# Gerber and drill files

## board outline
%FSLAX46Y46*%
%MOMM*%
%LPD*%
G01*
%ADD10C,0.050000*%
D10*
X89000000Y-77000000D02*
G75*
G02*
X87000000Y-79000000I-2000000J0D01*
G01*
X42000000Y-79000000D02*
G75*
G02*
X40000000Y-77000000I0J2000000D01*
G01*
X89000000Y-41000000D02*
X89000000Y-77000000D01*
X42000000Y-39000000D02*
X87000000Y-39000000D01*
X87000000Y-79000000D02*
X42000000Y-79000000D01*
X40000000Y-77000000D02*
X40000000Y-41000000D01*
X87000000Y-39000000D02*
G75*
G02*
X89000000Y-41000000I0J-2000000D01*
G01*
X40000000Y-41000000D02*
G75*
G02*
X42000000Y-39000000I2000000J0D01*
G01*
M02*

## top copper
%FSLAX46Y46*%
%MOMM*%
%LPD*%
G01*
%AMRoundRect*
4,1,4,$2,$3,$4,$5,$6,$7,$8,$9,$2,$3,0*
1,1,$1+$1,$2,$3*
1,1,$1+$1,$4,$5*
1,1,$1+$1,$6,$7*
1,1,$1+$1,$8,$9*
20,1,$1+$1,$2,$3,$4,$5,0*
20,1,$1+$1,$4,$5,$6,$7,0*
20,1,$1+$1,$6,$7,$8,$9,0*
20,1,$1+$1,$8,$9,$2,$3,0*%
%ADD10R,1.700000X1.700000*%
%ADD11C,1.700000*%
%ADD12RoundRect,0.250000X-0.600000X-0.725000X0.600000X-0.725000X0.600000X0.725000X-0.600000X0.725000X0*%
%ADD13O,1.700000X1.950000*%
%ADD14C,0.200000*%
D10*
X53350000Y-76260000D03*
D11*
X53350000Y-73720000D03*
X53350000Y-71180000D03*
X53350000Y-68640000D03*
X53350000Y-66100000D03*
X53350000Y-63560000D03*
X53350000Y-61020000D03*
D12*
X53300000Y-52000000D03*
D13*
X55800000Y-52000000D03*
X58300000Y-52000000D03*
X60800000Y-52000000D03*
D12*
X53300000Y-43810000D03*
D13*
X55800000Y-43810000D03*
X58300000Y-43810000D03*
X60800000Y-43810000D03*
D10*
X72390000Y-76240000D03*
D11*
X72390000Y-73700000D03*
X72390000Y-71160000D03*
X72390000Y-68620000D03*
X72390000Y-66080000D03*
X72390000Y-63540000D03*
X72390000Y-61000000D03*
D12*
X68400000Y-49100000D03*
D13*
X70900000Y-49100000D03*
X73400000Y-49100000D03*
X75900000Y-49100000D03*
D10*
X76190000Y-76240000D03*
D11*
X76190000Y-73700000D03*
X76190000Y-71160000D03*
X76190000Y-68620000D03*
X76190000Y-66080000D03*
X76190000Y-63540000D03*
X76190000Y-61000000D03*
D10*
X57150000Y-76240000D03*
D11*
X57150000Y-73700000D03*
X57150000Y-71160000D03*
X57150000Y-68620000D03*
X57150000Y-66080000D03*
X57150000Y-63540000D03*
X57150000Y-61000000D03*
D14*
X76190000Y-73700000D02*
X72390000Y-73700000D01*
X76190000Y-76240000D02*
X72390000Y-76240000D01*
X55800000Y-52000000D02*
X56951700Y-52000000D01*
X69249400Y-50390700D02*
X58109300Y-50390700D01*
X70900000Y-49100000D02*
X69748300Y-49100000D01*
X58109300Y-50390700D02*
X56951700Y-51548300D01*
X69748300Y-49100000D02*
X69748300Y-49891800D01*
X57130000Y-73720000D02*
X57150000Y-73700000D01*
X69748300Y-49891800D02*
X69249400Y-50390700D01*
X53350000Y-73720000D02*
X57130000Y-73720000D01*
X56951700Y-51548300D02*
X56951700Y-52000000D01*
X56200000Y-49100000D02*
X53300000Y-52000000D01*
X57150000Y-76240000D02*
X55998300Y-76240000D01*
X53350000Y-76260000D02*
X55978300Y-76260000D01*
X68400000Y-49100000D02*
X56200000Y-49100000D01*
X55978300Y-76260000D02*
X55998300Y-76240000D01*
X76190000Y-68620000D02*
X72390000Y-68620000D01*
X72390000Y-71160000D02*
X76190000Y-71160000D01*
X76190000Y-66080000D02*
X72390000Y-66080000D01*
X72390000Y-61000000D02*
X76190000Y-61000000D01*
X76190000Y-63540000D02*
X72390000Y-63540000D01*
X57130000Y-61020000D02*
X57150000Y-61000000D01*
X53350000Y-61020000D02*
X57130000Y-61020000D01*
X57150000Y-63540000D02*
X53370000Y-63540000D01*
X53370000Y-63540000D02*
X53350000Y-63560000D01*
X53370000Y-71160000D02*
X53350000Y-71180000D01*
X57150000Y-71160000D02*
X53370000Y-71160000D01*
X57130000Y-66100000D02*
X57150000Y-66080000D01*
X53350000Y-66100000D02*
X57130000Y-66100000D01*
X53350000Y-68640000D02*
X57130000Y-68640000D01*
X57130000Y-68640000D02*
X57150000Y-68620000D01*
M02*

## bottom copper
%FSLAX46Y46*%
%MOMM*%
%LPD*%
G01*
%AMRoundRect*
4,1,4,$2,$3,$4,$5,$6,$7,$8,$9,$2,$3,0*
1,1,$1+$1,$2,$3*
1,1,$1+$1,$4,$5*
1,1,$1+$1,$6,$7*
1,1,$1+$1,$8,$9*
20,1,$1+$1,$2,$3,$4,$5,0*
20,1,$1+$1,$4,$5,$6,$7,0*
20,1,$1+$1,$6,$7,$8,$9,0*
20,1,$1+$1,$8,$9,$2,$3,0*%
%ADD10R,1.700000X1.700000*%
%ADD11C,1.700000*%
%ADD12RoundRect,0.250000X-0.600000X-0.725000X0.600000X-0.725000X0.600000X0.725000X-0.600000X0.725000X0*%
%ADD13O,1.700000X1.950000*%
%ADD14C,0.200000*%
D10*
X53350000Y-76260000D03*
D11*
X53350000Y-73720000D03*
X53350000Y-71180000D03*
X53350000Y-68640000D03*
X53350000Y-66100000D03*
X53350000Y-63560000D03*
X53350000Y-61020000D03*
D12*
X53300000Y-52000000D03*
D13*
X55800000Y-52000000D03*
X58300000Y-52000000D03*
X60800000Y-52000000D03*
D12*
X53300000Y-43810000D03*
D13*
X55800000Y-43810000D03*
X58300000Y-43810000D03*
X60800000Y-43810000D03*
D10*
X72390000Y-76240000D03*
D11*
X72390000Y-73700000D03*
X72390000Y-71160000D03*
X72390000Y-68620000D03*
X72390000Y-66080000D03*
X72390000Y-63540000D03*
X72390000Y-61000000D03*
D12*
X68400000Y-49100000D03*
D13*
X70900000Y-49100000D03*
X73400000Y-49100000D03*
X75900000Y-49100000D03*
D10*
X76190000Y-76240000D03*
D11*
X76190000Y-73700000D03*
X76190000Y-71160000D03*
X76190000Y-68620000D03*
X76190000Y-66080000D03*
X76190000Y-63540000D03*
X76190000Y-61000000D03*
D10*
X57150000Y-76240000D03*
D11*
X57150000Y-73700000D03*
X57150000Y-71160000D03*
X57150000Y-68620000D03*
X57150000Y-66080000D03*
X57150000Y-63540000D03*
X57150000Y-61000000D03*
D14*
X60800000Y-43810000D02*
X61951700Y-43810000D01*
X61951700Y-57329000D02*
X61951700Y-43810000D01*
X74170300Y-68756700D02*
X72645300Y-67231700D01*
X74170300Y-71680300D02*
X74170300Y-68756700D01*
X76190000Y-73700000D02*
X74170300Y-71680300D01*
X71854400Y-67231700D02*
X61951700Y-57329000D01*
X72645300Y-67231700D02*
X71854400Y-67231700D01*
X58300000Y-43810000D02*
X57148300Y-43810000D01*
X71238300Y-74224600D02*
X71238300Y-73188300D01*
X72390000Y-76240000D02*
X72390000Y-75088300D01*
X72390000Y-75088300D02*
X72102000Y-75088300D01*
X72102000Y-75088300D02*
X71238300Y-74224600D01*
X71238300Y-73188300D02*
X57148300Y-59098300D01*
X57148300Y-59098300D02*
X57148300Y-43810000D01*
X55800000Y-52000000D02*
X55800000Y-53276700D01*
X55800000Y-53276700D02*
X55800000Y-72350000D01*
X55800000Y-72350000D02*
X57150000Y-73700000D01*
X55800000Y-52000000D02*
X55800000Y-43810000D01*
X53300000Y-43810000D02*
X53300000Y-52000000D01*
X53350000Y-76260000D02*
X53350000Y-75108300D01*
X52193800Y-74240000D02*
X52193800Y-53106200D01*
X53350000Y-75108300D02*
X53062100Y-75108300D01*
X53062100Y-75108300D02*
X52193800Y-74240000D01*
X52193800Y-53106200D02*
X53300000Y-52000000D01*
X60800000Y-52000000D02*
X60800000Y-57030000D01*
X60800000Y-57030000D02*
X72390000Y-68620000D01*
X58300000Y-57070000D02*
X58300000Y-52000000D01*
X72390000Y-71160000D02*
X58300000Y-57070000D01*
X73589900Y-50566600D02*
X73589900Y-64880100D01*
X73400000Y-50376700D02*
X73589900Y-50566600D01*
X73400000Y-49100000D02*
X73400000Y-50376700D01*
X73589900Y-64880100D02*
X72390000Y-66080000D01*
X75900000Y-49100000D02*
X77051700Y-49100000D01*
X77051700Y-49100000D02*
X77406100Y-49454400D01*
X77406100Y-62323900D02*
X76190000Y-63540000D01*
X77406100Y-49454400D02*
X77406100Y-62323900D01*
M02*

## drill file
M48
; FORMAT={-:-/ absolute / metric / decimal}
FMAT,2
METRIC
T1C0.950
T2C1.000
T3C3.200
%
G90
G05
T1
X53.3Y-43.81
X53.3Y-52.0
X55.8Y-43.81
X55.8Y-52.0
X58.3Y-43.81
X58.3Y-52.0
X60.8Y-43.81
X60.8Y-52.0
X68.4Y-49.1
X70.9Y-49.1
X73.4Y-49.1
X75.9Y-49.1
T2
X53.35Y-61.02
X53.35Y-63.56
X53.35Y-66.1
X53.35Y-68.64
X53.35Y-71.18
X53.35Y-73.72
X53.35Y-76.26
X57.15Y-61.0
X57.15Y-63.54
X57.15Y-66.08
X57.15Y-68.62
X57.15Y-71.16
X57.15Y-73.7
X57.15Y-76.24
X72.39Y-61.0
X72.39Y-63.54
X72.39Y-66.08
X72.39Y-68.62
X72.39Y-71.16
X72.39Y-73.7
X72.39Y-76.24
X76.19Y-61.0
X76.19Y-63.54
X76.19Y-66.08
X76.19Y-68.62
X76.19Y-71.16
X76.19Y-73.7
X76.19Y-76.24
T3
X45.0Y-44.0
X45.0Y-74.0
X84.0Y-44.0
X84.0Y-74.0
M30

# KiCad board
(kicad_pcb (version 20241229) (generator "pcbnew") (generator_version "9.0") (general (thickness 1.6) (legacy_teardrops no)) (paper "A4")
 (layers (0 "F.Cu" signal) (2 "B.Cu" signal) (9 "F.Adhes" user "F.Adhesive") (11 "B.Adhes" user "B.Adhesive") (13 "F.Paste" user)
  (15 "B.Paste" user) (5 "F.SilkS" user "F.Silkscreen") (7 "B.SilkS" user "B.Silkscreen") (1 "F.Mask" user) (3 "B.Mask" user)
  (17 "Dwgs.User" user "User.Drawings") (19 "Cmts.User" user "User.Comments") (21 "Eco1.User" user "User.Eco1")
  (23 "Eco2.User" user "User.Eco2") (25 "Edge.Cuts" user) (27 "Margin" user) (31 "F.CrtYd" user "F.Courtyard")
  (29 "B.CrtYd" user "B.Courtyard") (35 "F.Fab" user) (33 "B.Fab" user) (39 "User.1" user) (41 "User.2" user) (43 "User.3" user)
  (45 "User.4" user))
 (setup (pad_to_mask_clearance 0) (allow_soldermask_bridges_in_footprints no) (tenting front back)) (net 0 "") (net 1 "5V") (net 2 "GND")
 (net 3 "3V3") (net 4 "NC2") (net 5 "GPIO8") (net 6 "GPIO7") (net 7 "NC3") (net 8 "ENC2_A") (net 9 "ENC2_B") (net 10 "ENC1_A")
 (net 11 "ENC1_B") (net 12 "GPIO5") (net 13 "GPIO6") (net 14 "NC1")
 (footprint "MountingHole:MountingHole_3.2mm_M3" (layer "F.Cu") (at 84 44)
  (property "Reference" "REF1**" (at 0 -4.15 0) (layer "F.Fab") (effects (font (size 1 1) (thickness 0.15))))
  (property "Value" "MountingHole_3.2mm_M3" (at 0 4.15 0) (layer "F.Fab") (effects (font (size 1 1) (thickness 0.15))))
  (pad "" np_thru_hole circle (at 0 0) (size 3.2 3.2) (drill 3.2) (layers "*.Cu" "*.Mask")))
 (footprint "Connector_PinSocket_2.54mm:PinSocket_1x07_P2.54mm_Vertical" (layer "F.Cu") (at 53.35 76.26 180)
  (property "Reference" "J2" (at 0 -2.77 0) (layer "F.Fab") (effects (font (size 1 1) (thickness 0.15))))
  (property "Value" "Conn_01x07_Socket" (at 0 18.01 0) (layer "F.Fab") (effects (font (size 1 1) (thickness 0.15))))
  (pad "1" thru_hole rect (at 0 0 180) (size 1.7 1.7) (drill 1) (layers "*.Cu" "*.Mask") (remove_unused_layers no) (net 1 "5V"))
  (pad "2" thru_hole circle (at 0 2.54 180) (size 1.7 1.7) (drill 1) (layers "*.Cu" "*.Mask") (remove_unused_layers no) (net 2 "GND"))
  (pad "3" thru_hole circle (at 0 5.08 180) (size 1.7 1.7) (drill 1) (layers "*.Cu" "*.Mask") (remove_unused_layers no) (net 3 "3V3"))
  (pad "4" thru_hole circle (at 0 7.62 180) (size 1.7 1.7) (drill 1) (layers "*.Cu" "*.Mask") (remove_unused_layers no) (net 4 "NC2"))
  (pad "5" thru_hole circle (at 0 10.16 180) (size 1.7 1.7) (drill 1) (layers "*.Cu" "*.Mask") (remove_unused_layers no) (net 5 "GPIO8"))
  (pad "6" thru_hole circle (at 0 12.7 180) (size 1.7 1.7) (drill 1) (layers "*.Cu" "*.Mask") (remove_unused_layers no) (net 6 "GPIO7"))
  (pad "7" thru_hole circle (at 0 15.24 180) (size 1.7 1.7) (drill 1) (layers "*.Cu" "*.Mask") (remove_unused_layers no) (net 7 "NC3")))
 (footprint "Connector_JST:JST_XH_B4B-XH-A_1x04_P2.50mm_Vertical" (layer "F.Cu") (at 53.3 52)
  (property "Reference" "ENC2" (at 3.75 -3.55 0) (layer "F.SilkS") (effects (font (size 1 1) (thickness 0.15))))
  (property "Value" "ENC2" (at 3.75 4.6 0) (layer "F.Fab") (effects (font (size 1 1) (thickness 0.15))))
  (pad "1" thru_hole roundrect (at 0 0) (size 1.7 1.95) (drill 0.95) (layers "*.Cu" "*.Mask") (remove_unused_layers no)
   (roundrect_rratio 0.147059) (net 1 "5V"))
  (pad "2" thru_hole oval (at 2.5 0) (size 1.7 1.95) (drill 0.95) (layers "*.Cu" "*.Mask") (remove_unused_layers no) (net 2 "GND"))
  (pad "3" thru_hole oval (at 5 0) (size 1.7 1.95) (drill 0.95) (layers "*.Cu" "*.Mask") (remove_unused_layers no) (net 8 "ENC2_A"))
  (pad "4" thru_hole oval (at 7.5 0) (size 1.7 1.95) (drill 0.95) (layers "*.Cu" "*.Mask") (remove_unused_layers no) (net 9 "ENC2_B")))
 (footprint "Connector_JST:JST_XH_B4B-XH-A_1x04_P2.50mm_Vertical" (layer "F.Cu") (at 53.3 43.81)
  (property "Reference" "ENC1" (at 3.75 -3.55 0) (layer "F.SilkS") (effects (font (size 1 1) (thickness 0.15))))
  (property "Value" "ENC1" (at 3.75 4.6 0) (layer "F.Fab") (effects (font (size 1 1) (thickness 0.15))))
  (pad "1" thru_hole roundrect (at 0 0) (size 1.7 1.95) (drill 0.95) (layers "*.Cu" "*.Mask") (remove_unused_layers no)
   (roundrect_rratio 0.147059) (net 1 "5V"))
  (pad "2" thru_hole oval (at 2.5 0) (size 1.7 1.95) (drill 0.95) (layers "*.Cu" "*.Mask") (remove_unused_layers no) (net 2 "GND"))
  (pad "3" thru_hole oval (at 5 0) (size 1.7 1.95) (drill 0.95) (layers "*.Cu" "*.Mask") (remove_unused_layers no) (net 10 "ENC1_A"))
  (pad "4" thru_hole oval (at 7.5 0) (size 1.7 1.95) (drill 0.95) (layers "*.Cu" "*.Mask") (remove_unused_layers no) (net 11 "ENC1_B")))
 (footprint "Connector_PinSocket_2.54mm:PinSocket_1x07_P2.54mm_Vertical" (layer "F.Cu") (at 72.39 76.24 180)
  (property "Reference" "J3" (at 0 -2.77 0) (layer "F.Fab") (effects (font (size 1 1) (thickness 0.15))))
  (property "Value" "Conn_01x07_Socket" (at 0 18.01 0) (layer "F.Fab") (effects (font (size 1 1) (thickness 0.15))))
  (pad "1" thru_hole rect (at 0 0 180) (size 1.7 1.7) (drill 1) (layers "*.Cu" "*.Mask") (remove_unused_layers no) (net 10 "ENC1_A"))
  (pad "2" thru_hole circle (at 0 2.54 180) (size 1.7 1.7) (drill 1) (layers "*.Cu" "*.Mask") (remove_unused_layers no) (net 11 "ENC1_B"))
  (pad "3" thru_hole circle (at 0 5.08 180) (size 1.7 1.7) (drill 1) (layers "*.Cu" "*.Mask") (remove_unused_layers no) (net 8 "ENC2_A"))
  (pad "4" thru_hole circle (at 0 7.62 180) (size 1.7 1.7) (drill 1) (layers "*.Cu" "*.Mask") (remove_unused_layers no) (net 9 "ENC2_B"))
  (pad "5" thru_hole circle (at 0 10.16 180) (size 1.7 1.7) (drill 1) (layers "*.Cu" "*.Mask") (remove_unused_layers no) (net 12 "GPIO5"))
  (pad "6" thru_hole circle (at 0 12.7 180) (size 1.7 1.7) (drill 1) (layers "*.Cu" "*.Mask") (remove_unused_layers no) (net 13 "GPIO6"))
  (pad "7" thru_hole circle (at 0 15.24 180) (size 1.7 1.7) (drill 1) (layers "*.Cu" "*.Mask") (remove_unused_layers no) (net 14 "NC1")))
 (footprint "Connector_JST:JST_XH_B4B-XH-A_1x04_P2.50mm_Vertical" (layer "F.Cu") (at 68.4 49.1)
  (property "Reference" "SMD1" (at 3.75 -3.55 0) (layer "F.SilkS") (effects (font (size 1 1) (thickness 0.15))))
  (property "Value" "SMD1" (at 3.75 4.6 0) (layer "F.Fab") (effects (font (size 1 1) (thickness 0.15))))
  (pad "1" thru_hole roundrect (at 0 0) (size 1.7 1.95) (drill 0.95) (layers "*.Cu" "*.Mask") (remove_unused_layers no)
   (roundrect_rratio 0.147059) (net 1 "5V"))
  (pad "2" thru_hole oval (at 2.5 0) (size 1.7 1.95) (drill 0.95) (layers "*.Cu" "*.Mask") (remove_unused_layers no) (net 2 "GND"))
  (pad "3" thru_hole oval (at 5 0) (size 1.7 1.95) (drill 0.95) (layers "*.Cu" "*.Mask") (remove_unused_layers no) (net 12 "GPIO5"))
  (pad "4" thru_hole oval (at 7.5 0) (size 1.7 1.95) (drill 0.95) (layers "*.Cu" "*.Mask") (remove_unused_layers no) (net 13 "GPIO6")))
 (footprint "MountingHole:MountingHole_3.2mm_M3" (layer "F.Cu") (at 45 74)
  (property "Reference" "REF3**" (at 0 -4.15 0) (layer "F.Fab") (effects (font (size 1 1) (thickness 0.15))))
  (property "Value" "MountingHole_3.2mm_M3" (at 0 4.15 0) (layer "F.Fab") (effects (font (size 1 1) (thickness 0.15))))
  (pad "" np_thru_hole circle (at 0 0) (size 3.2 3.2) (drill 3.2) (layers "*.Cu" "*.Mask")))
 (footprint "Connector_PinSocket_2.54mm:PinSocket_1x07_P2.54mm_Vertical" (layer "F.Cu") (at 76.19 76.24 180)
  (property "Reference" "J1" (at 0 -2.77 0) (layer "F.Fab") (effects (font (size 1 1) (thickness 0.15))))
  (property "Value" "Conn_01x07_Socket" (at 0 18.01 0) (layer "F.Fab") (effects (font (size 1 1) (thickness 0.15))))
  (pad "1" thru_hole rect (at 0 0 180) (size 1.7 1.7) (drill 1) (layers "*.Cu" "*.Mask") (remove_unused_layers no) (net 10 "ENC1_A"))
  (pad "2" thru_hole circle (at 0 2.54 180) (size 1.7 1.7) (drill 1) (layers "*.Cu" "*.Mask") (remove_unused_layers no) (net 11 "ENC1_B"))
  (pad "3" thru_hole circle (at 0 5.08 180) (size 1.7 1.7) (drill 1) (layers "*.Cu" "*.Mask") (remove_unused_layers no) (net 8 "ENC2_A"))
  (pad "4" thru_hole circle (at 0 7.62 180) (size 1.7 1.7) (drill 1) (layers "*.Cu" "*.Mask") (remove_unused_layers no) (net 9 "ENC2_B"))
  (pad "5" thru_hole circle (at 0 10.16 180) (size 1.7 1.7) (drill 1) (layers "*.Cu" "*.Mask") (remove_unused_layers no) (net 12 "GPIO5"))
  (pad "6" thru_hole circle (at 0 12.7 180) (size 1.7 1.7) (drill 1) (layers "*.Cu" "*.Mask") (remove_unused_layers no) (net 13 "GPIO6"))
  (pad "7" thru_hole circle (at 0 15.24 180) (size 1.7 1.7) (drill 1) (layers "*.Cu" "*.Mask") (remove_unused_layers no) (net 14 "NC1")))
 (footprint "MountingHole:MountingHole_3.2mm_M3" (layer "F.Cu") (at 45 44)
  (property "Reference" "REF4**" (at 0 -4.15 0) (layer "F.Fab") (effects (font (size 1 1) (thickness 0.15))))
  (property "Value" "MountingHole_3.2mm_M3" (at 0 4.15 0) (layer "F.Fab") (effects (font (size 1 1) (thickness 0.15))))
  (pad "" np_thru_hole circle (at 0 0) (size 3.2 3.2) (drill 3.2) (layers "*.Cu" "*.Mask")))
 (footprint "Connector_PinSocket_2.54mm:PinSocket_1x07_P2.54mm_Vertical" (layer "F.Cu") (at 57.15 76.24 180)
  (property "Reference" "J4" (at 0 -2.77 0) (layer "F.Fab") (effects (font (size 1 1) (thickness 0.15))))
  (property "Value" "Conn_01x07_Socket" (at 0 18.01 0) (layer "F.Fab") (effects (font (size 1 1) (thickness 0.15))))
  (pad "1" thru_hole rect (at 0 0 180) (size 1.7 1.7) (drill 1) (layers "*.Cu" "*.Mask") (remove_unused_layers no) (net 1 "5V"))
  (pad "2" thru_hole circle (at 0 2.54 180) (size 1.7 1.7) (drill 1) (layers "*.Cu" "*.Mask") (remove_unused_layers no) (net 2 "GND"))
  (pad "3" thru_hole circle (at 0 5.08 180) (size 1.7 1.7) (drill 1) (layers "*.Cu" "*.Mask") (remove_unused_layers no) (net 3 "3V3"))
  (pad "4" thru_hole circle (at 0 7.62 180) (size 1.7 1.7) (drill 1) (layers "*.Cu" "*.Mask") (remove_unused_layers no) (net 4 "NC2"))
  (pad "5" thru_hole circle (at 0 10.16 180) (size 1.7 1.7) (drill 1) (layers "*.Cu" "*.Mask") (remove_unused_layers no) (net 5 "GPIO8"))
  (pad "6" thru_hole circle (at 0 12.7 180) (size 1.7 1.7) (drill 1) (layers "*.Cu" "*.Mask") (remove_unused_layers no) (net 6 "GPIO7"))
  (pad "7" thru_hole circle (at 0 15.24 180) (size 1.7 1.7) (drill 1) (layers "*.Cu" "*.Mask") (remove_unused_layers no) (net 7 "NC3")))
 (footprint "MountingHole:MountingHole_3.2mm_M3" (layer "F.Cu") (at 84 74)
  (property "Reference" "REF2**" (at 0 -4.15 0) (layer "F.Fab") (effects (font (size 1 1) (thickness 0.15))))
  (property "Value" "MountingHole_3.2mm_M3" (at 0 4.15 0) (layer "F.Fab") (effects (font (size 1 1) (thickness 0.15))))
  (pad "" np_thru_hole circle (at 0 0) (size 3.2 3.2) (drill 3.2) (layers "*.Cu" "*.Mask")))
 (gr_arc (start 89 77) (mid 88.414214 78.414214) (end 87 79) (stroke (width 0.05) (type default)) (layer "Edge.Cuts"))
 (gr_arc (start 42 79) (mid 40.585786 78.414214) (end 40 77) (stroke (width 0.05) (type default)) (layer "Edge.Cuts"))
 (gr_line (start 89 41) (end 89 77) (stroke (width 0.05) (type default)) (layer "Edge.Cuts"))
 (gr_line (start 42 39) (end 87 39) (stroke (width 0.05) (type default)) (layer "Edge.Cuts"))
 (gr_line (start 87 79) (end 42 79) (stroke (width 0.05) (type default)) (layer "Edge.Cuts"))
 (gr_line (start 40 77) (end 40 41) (stroke (width 0.05) (type default)) (layer "Edge.Cuts"))
 (gr_arc (start 87 39) (mid 88.414214 39.585786) (end 89 41) (stroke (width 0.05) (type default)) (layer "Edge.Cuts"))
 (gr_arc (start 40 41) (mid 40.585786 39.585786) (end 42 39) (stroke (width 0.05) (type default)) (layer "Edge.Cuts"))
 (segment (start 76.19 73.7) (end 72.39 73.7) (width 0.2) (layer "F.Cu") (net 11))
 (segment (start 60.8 43.81) (end 61.9517 43.81) (width 0.2) (layer "B.Cu") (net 11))
 (segment (start 61.9517 57.329) (end 61.9517 43.81) (width 0.2) (layer "B.Cu") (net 11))
 (segment (start 74.1703 68.7567) (end 72.6453 67.2317) (width 0.2) (layer "B.Cu") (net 11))
 (segment (start 74.1703 71.6803) (end 74.1703 68.7567) (width 0.2) (layer "B.Cu") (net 11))
 (segment (start 76.19 73.7) (end 74.1703 71.6803) (width 0.2) (layer "B.Cu") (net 11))
 (segment (start 71.8544 67.2317) (end 61.9517 57.329) (width 0.2) (layer "B.Cu") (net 11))
 (segment (start 72.6453 67.2317) (end 71.8544 67.2317) (width 0.2) (layer "B.Cu") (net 11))
 (segment (start 76.19 76.24) (end 72.39 76.24) (width 0.2) (layer "F.Cu") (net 10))
 (segment (start 58.3 43.81) (end 57.1483 43.81) (width 0.2) (layer "B.Cu") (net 10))
 (segment (start 71.2383 74.2246) (end 71.2383 73.1883) (width 0.2) (layer "B.Cu") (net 10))
 (segment (start 72.39 76.24) (end 72.39 75.0883) (width 0.2) (layer "B.Cu") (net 10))
 (segment (start 72.39 75.0883) (end 72.102 75.0883) (width 0.2) (layer "B.Cu") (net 10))
 (segment (start 72.102 75.0883) (end 71.2383 74.2246) (width 0.2) (layer "B.Cu") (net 10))
 (segment (start 71.2383 73.1883) (end 57.1483 59.0983) (width 0.2) (layer "B.Cu") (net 10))
 (segment (start 57.1483 59.0983) (end 57.1483 43.81) (width 0.2) (layer "B.Cu") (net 10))
 (segment (start 55.8 52) (end 56.9517 52) (width 0.2) (layer "F.Cu") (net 2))
 (segment (start 69.2494 50.3907) (end 58.1093 50.3907) (width 0.2) (layer "F.Cu") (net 2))
 (segment (start 70.9 49.1) (end 69.7483 49.1) (width 0.2) (layer "F.Cu") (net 2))
 (segment (start 58.1093 50.3907) (end 56.9517 51.5483) (width 0.2) (layer "F.Cu") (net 2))
 (segment (start 69.7483 49.1) (end 69.7483 49.8918) (width 0.2) (layer "F.Cu") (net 2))
 (segment (start 57.13 73.72) (end 57.15 73.7) (width 0.2) (layer "F.Cu") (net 2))
 (segment (start 69.7483 49.8918) (end 69.2494 50.3907) (width 0.2) (layer "F.Cu") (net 2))
 (segment (start 53.35 73.72) (end 57.13 73.72) (width 0.2) (layer "F.Cu") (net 2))
 (segment (start 56.9517 51.5483) (end 56.9517 52) (width 0.2) (layer "F.Cu") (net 2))
 (segment (start 55.8 52) (end 55.8 53.2767) (width 0.2) (layer "B.Cu") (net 2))
 (segment (start 55.8 53.2767) (end 55.8 72.35) (width 0.2) (layer "B.Cu") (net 2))
 (segment (start 55.8 72.35) (end 57.15 73.7) (width 0.2) (layer "B.Cu") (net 2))
 (segment (start 55.8 52) (end 55.8 43.81) (width 0.2) (layer "B.Cu") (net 2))
 (segment (start 56.2 49.1) (end 53.3 52) (width 0.2) (layer "F.Cu") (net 1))
 (segment (start 57.15 76.24) (end 55.9983 76.24) (width 0.2) (layer "F.Cu") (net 1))
 (segment (start 53.35 76.26) (end 55.9783 76.26) (width 0.2) (layer "F.Cu") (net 1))
 (segment (start 68.4 49.1) (end 56.2 49.1) (width 0.2) (layer "F.Cu") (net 1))
 (segment (start 55.9783 76.26) (end 55.9983 76.24) (width 0.2) (layer "F.Cu") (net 1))
 (segment (start 53.3 43.81) (end 53.3 52) (width 0.2) (layer "B.Cu") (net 1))
 (segment (start 53.35 76.26) (end 53.35 75.1083) (width 0.2) (layer "B.Cu") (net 1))
 (segment (start 52.1938 74.24) (end 52.1938 53.1062) (width 0.2) (layer "B.Cu") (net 1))
 (segment (start 53.35 75.1083) (end 53.0621 75.1083) (width 0.2) (layer "B.Cu") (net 1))
 (segment (start 53.0621 75.1083) (end 52.1938 74.24) (width 0.2) (layer "B.Cu") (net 1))
 (segment (start 52.1938 53.1062) (end 53.3 52) (width 0.2) (layer "B.Cu") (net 1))
 (segment (start 76.19 68.62) (end 72.39 68.62) (width 0.2) (layer "F.Cu") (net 9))
 (segment (start 60.8 52) (end 60.8 57.03) (width 0.2) (layer "B.Cu") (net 9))
 (segment (start 60.8 57.03) (end 72.39 68.62) (width 0.2) (layer "B.Cu") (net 9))
 (segment (start 72.39 71.16) (end 76.19 71.16) (width 0.2) (layer "F.Cu") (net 8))
 (segment (start 58.3 57.07) (end 58.3 52) (width 0.2) (layer "B.Cu") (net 8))
 (segment (start 72.39 71.16) (end 58.3 57.07) (width 0.2) (layer "B.Cu") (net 8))
 (segment (start 76.19 66.08) (end 72.39 66.08) (width 0.2) (layer "F.Cu") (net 12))
 (segment (start 73.5899 50.5666) (end 73.5899 64.8801) (width 0.2) (layer "B.Cu") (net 12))
 (segment (start 73.4 50.3767) (end 73.5899 50.5666) (width 0.2) (layer "B.Cu") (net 12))
 (segment (start 73.4 49.1) (end 73.4 50.3767) (width 0.2) (layer "B.Cu") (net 12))
 (segment (start 73.5899 64.8801) (end 72.39 66.08) (width 0.2) (layer "B.Cu") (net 12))
 (segment (start 72.39 61) (end 76.19 61) (width 0.2) (layer "F.Cu") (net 14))
 (segment (start 76.19 63.54) (end 72.39 63.54) (width 0.2) (layer "F.Cu") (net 13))
 (segment (start 75.9 49.1) (end 77.0517 49.1) (width 0.2) (layer "B.Cu") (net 13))
 (segment (start 77.0517 49.1) (end 77.4061 49.4544) (width 0.2) (layer "B.Cu") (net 13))
 (segment (start 77.4061 62.3239) (end 76.19 63.54) (width 0.2) (layer "B.Cu") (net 13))
 (segment (start 77.4061 49.4544) (end 77.4061 62.3239) (width 0.2) (layer "B.Cu") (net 13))
 (segment (start 57.13 61.02) (end 57.15 61) (width 0.2) (layer "F.Cu") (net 7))
 (segment (start 53.35 61.02) (end 57.13 61.02) (width 0.2) (layer "F.Cu") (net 7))
 (segment (start 57.15 63.54) (end 53.37 63.54) (width 0.2) (layer "F.Cu") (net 6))
 (segment (start 53.37 63.54) (end 53.35 63.56) (width 0.2) (layer "F.Cu") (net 6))
 (segment (start 53.37 71.16) (end 53.35 71.18) (width 0.2) (layer "F.Cu") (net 3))
 (segment (start 57.15 71.16) (end 53.37 71.16) (width 0.2) (layer "F.Cu") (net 3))
 (segment (start 57.13 66.1) (end 57.15 66.08) (width 0.2) (layer "F.Cu") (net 5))
 (segment (start 53.35 66.1) (end 57.13 66.1) (width 0.2) (layer "F.Cu") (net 5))
 (segment (start 53.35 68.64) (end 57.13 68.64) (width 0.2) (layer "F.Cu") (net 4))
 (segment (start 57.13 68.64) (end 57.15 68.62) (width 0.2) (layer "F.Cu") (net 4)))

